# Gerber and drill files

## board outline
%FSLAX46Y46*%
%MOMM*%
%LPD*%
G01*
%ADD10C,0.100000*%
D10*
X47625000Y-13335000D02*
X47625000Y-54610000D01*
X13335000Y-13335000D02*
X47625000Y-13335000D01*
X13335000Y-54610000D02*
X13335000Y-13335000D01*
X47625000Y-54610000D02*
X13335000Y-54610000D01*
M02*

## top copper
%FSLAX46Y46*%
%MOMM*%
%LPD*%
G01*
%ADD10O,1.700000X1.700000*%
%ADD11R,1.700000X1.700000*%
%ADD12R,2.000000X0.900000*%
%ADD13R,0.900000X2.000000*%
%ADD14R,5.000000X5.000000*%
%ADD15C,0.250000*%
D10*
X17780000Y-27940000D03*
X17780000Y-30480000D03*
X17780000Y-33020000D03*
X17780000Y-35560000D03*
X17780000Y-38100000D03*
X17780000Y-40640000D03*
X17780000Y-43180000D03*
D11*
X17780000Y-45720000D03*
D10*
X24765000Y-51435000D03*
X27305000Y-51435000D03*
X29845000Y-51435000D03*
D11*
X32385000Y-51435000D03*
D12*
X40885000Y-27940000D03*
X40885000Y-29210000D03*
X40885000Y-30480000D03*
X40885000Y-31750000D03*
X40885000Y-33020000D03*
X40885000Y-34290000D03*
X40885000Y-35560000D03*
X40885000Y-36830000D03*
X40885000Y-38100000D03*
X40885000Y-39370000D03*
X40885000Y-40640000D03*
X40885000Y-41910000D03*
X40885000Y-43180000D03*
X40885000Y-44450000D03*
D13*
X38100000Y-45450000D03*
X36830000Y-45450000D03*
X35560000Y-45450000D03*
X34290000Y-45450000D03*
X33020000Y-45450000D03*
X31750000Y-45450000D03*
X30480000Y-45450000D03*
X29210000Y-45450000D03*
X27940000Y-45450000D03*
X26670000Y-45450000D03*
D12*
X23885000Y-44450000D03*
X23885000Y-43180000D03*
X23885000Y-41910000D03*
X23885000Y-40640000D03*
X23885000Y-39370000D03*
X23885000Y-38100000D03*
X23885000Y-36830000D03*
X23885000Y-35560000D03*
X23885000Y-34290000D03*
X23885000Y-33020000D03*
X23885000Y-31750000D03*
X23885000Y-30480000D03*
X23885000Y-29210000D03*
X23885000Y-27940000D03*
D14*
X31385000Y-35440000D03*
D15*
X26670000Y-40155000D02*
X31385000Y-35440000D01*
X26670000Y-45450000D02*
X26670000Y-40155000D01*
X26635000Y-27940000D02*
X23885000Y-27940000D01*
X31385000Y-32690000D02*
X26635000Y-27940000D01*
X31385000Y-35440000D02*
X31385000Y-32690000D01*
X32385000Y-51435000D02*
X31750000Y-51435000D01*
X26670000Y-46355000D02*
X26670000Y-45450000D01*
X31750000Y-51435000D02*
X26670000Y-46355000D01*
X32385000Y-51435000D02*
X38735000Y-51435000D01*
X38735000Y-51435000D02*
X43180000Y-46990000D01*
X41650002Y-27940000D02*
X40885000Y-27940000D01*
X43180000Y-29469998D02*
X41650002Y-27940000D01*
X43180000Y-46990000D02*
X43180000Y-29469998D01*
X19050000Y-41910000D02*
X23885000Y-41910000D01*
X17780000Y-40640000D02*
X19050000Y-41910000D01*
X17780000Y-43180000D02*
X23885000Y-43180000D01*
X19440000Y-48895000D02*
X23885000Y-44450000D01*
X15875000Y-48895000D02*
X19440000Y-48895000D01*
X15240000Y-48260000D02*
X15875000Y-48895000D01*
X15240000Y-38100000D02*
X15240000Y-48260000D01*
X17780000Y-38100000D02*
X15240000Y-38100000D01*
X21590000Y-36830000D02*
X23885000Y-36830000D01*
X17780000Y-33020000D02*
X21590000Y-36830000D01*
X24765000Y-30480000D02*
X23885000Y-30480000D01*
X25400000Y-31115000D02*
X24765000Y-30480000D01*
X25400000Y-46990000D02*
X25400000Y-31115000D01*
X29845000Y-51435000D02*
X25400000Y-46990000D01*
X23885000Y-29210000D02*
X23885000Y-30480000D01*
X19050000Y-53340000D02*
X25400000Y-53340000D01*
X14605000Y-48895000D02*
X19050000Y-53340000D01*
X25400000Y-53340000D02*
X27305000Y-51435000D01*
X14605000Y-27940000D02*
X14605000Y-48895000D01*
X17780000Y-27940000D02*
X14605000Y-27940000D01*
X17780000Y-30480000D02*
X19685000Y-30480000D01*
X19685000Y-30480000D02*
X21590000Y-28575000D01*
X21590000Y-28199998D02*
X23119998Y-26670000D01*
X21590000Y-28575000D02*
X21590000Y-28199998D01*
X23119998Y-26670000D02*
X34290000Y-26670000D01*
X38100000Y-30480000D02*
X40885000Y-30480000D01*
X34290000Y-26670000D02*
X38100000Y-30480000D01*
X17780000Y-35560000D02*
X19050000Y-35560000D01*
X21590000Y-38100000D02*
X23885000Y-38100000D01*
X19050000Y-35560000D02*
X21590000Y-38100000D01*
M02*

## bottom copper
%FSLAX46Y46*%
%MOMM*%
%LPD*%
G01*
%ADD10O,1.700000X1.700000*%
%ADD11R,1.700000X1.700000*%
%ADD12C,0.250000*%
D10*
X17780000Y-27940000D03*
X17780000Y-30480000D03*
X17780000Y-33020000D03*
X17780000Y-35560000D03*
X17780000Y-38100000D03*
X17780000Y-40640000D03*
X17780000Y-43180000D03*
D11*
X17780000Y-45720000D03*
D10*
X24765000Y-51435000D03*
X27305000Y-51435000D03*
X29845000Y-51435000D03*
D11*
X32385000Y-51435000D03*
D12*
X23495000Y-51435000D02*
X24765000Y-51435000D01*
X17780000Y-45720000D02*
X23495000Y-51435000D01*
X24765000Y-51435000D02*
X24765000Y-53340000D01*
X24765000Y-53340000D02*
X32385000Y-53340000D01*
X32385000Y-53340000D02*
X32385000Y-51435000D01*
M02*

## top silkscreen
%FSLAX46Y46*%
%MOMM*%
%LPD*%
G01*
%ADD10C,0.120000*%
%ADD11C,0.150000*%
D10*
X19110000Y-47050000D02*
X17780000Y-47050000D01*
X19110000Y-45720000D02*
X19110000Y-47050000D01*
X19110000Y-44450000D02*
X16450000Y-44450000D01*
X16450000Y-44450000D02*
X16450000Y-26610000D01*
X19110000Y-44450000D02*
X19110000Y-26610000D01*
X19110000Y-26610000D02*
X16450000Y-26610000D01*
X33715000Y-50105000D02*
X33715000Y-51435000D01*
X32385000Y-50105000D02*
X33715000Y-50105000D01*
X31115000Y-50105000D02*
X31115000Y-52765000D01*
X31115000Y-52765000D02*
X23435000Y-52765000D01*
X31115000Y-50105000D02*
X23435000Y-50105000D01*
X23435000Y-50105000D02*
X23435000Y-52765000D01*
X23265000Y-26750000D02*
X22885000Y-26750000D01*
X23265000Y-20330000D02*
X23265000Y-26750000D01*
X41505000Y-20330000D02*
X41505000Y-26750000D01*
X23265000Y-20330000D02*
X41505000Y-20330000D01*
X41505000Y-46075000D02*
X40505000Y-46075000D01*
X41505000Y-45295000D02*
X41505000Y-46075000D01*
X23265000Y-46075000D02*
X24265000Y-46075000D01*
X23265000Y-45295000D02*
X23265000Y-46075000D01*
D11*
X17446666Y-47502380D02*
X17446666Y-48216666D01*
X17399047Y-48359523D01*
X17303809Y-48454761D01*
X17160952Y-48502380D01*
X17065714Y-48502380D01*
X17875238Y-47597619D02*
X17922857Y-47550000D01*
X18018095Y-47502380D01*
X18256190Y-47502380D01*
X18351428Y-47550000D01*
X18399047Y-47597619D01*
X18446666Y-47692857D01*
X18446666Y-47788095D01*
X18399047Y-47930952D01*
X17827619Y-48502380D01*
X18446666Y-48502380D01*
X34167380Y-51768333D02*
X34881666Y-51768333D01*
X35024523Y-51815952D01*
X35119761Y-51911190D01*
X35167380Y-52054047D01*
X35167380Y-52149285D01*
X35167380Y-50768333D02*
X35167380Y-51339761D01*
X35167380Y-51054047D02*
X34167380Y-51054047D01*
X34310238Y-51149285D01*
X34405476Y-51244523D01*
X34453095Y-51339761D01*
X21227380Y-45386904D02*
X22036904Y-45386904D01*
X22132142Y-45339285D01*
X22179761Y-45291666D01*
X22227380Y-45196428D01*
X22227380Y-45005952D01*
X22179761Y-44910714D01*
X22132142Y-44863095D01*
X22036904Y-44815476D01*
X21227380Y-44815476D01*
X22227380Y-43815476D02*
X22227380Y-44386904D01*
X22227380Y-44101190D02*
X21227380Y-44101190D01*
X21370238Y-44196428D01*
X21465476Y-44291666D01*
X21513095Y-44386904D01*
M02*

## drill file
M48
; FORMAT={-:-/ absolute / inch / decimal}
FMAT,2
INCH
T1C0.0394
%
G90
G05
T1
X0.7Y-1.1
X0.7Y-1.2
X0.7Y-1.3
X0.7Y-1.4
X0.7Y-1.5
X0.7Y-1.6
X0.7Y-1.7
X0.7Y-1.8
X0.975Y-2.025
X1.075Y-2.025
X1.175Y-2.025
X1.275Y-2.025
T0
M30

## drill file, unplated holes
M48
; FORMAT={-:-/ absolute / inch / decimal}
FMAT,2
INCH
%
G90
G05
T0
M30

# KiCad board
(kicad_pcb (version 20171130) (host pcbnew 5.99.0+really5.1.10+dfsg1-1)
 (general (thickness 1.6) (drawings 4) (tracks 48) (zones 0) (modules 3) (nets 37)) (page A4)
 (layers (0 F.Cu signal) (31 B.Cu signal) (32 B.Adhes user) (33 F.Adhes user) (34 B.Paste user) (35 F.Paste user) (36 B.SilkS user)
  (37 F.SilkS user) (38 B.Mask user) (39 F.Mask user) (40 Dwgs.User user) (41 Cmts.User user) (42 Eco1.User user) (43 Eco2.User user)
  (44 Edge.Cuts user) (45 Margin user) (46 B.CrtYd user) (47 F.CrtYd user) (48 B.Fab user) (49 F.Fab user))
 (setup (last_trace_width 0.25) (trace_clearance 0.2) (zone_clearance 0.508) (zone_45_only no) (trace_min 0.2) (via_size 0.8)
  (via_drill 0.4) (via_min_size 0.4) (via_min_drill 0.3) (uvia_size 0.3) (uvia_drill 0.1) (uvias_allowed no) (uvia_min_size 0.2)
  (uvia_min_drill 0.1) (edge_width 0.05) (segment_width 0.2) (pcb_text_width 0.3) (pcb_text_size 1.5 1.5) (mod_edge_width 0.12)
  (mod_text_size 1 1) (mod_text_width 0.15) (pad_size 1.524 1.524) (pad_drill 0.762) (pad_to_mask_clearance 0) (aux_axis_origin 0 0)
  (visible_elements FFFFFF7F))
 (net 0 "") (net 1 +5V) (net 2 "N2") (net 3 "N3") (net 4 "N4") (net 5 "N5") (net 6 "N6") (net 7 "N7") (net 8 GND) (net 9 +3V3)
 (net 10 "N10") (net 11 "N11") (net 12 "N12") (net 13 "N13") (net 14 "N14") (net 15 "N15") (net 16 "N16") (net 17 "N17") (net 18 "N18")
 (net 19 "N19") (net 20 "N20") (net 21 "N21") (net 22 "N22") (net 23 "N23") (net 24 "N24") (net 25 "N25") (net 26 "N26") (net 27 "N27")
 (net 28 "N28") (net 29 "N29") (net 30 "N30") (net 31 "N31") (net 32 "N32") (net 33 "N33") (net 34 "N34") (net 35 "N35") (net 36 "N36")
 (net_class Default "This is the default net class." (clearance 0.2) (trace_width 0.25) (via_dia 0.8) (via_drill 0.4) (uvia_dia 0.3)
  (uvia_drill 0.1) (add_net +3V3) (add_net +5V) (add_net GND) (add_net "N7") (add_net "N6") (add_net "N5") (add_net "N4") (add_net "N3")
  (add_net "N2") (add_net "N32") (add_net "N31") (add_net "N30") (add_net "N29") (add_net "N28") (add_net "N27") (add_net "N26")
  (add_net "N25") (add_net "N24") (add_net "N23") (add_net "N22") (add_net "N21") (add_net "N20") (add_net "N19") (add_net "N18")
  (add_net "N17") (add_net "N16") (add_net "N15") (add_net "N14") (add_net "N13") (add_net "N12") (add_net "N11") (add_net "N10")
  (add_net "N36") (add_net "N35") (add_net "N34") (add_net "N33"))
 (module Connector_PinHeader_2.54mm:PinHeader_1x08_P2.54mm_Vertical (layer F.Cu) (at 17.78 45.72 180)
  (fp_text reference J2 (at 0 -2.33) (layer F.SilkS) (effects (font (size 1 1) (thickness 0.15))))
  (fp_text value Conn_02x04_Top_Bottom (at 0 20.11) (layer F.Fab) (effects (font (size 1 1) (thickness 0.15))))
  (fp_line (start -1.33 -1.33) (end 0 -1.33) (layer F.SilkS) (width 0.12))
  (fp_line (start -1.33 0) (end -1.33 -1.33) (layer F.SilkS) (width 0.12))
  (fp_line (start -1.33 1.27) (end 1.33 1.27) (layer F.SilkS) (width 0.12))
  (fp_line (start 1.33 1.27) (end 1.33 19.11) (layer F.SilkS) (width 0.12))
  (fp_line (start -1.33 1.27) (end -1.33 19.11) (layer F.SilkS) (width 0.12))
  (fp_line (start -1.33 19.11) (end 1.33 19.11) (layer F.SilkS) (width 0.12))
  (pad 8 thru_hole oval (at 0 17.78 180) (size 1.7 1.7) (drill 1) (layers *.Cu *.Mask) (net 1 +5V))
  (pad 7 thru_hole oval (at 0 15.24 180) (size 1.7 1.7) (drill 1) (layers *.Cu *.Mask) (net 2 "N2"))
  (pad 6 thru_hole oval (at 0 12.7 180) (size 1.7 1.7) (drill 1) (layers *.Cu *.Mask) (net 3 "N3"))
  (pad 5 thru_hole oval (at 0 10.16 180) (size 1.7 1.7) (drill 1) (layers *.Cu *.Mask) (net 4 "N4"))
  (pad 4 thru_hole oval (at 0 7.62 180) (size 1.7 1.7) (drill 1) (layers *.Cu *.Mask) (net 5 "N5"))
  (pad 3 thru_hole oval (at 0 5.08 180) (size 1.7 1.7) (drill 1) (layers *.Cu *.Mask) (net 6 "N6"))
  (pad 2 thru_hole oval (at 0 2.54 180) (size 1.7 1.7) (drill 1) (layers *.Cu *.Mask) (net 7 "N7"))
  (pad 1 thru_hole rect (at 0 0 180) (size 1.7 1.7) (drill 1) (layers *.Cu *.Mask) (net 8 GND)))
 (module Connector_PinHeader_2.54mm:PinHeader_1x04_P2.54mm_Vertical (layer F.Cu) (at 32.385 51.435 270)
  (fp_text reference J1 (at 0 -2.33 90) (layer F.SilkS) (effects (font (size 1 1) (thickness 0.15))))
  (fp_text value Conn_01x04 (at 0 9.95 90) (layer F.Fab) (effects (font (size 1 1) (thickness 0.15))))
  (fp_line (start -1.33 -1.33) (end 0 -1.33) (layer F.SilkS) (width 0.12))
  (fp_line (start -1.33 0) (end -1.33 -1.33) (layer F.SilkS) (width 0.12))
  (fp_line (start -1.33 1.27) (end 1.33 1.27) (layer F.SilkS) (width 0.12))
  (fp_line (start 1.33 1.27) (end 1.33 8.95) (layer F.SilkS) (width 0.12))
  (fp_line (start -1.33 1.27) (end -1.33 8.95) (layer F.SilkS) (width 0.12))
  (fp_line (start -1.33 8.95) (end 1.33 8.95) (layer F.SilkS) (width 0.12))
  (pad 4 thru_hole oval (at 0 7.62 270) (size 1.7 1.7) (drill 1) (layers *.Cu *.Mask) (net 8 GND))
  (pad 3 thru_hole oval (at 0 5.08 270) (size 1.7 1.7) (drill 1) (layers *.Cu *.Mask) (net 1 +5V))
  (pad 2 thru_hole oval (at 0 2.54 270) (size 1.7 1.7) (drill 1) (layers *.Cu *.Mask) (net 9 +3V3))
  (pad 1 thru_hole rect (at 0 0 270) (size 1.7 1.7) (drill 1) (layers *.Cu *.Mask) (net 8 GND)))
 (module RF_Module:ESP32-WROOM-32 (layer F.Cu) (at 32.385 36.195)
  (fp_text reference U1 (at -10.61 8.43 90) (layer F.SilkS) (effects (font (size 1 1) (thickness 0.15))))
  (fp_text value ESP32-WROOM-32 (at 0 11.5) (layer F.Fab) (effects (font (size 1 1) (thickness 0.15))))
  (fp_line (start -9.12 -9.445) (end -9.5 -9.445) (layer F.SilkS) (width 0.12))
  (fp_line (start -9.12 -15.865) (end -9.12 -9.445) (layer F.SilkS) (width 0.12))
  (fp_line (start 9.12 -15.865) (end 9.12 -9.445) (layer F.SilkS) (width 0.12))
  (fp_line (start -9.12 -15.865) (end 9.12 -15.865) (layer F.SilkS) (width 0.12))
  (fp_line (start 9.12 9.88) (end 8.12 9.88) (layer F.SilkS) (width 0.12))
  (fp_line (start 9.12 9.1) (end 9.12 9.88) (layer F.SilkS) (width 0.12))
  (fp_line (start -9.12 9.88) (end -8.12 9.88) (layer F.SilkS) (width 0.12))
  (fp_line (start -9.12 9.1) (end -9.12 9.88) (layer F.SilkS) (width 0.12))
  (pad 38 smd rect (at 8.5 -8.255) (size 2 0.9) (layers F.Cu F.Paste F.Mask) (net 8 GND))
  (pad 37 smd rect (at 8.5 -6.985) (size 2 0.9) (layers F.Cu F.Paste F.Mask) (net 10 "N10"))
  (pad 36 smd rect (at 8.5 -5.715) (size 2 0.9) (layers F.Cu F.Paste F.Mask) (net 2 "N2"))
  (pad 35 smd rect (at 8.5 -4.445) (size 2 0.9) (layers F.Cu F.Paste F.Mask) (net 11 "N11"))
  (pad 34 smd rect (at 8.5 -3.175) (size 2 0.9) (layers F.Cu F.Paste F.Mask) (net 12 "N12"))
  (pad 33 smd rect (at 8.5 -1.905) (size 2 0.9) (layers F.Cu F.Paste F.Mask) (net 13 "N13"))
  (pad 32 smd rect (at 8.5 -0.635) (size 2 0.9) (layers F.Cu F.Paste F.Mask) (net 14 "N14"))
  (pad 31 smd rect (at 8.5 0.635) (size 2 0.9) (layers F.Cu F.Paste F.Mask) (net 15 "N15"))
  (pad 30 smd rect (at 8.5 1.905) (size 2 0.9) (layers F.Cu F.Paste F.Mask) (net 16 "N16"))
  (pad 29 smd rect (at 8.5 3.175) (size 2 0.9) (layers F.Cu F.Paste F.Mask) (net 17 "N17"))
  (pad 28 smd rect (at 8.5 4.445) (size 2 0.9) (layers F.Cu F.Paste F.Mask) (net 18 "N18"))
  (pad 27 smd rect (at 8.5 5.715) (size 2 0.9) (layers F.Cu F.Paste F.Mask) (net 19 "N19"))
  (pad 26 smd rect (at 8.5 6.985) (size 2 0.9) (layers F.Cu F.Paste F.Mask) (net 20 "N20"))
  (pad 25 smd rect (at 8.5 8.255) (size 2 0.9) (layers F.Cu F.Paste F.Mask) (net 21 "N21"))
  (pad 24 smd rect (at 5.715 9.255 90) (size 2 0.9) (layers F.Cu F.Paste F.Mask) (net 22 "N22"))
  (pad 23 smd rect (at 4.445 9.255 90) (size 2 0.9) (layers F.Cu F.Paste F.Mask) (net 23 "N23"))
  (pad 22 smd rect (at 3.175 9.255 90) (size 2 0.9) (layers F.Cu F.Paste F.Mask) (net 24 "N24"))
  (pad 21 smd rect (at 1.905 9.255 90) (size 2 0.9) (layers F.Cu F.Paste F.Mask) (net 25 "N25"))
  (pad 20 smd rect (at 0.635 9.255 90) (size 2 0.9) (layers F.Cu F.Paste F.Mask) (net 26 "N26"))
  (pad 19 smd rect (at -0.635 9.255 90) (size 2 0.9) (layers F.Cu F.Paste F.Mask) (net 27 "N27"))
  (pad 18 smd rect (at -1.905 9.255 90) (size 2 0.9) (layers F.Cu F.Paste F.Mask) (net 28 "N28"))
  (pad 17 smd rect (at -3.175 9.255 90) (size 2 0.9) (layers F.Cu F.Paste F.Mask) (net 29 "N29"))
  (pad 16 smd rect (at -4.445 9.255 90) (size 2 0.9) (layers F.Cu F.Paste F.Mask) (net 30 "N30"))
  (pad 15 smd rect (at -5.715 9.255 90) (size 2 0.9) (layers F.Cu F.Paste F.Mask) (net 8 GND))
  (pad 14 smd rect (at -8.5 8.255) (size 2 0.9) (layers F.Cu F.Paste F.Mask) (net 5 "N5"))
  (pad 13 smd rect (at -8.5 6.985) (size 2 0.9) (layers F.Cu F.Paste F.Mask) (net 7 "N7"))
  (pad 12 smd rect (at -8.5 5.715) (size 2 0.9) (layers F.Cu F.Paste F.Mask) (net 6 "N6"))
  (pad 11 smd rect (at -8.5 4.445) (size 2 0.9) (layers F.Cu F.Paste F.Mask) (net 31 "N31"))
  (pad 10 smd rect (at -8.5 3.175) (size 2 0.9) (layers F.Cu F.Paste F.Mask) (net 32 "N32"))
  (pad 9 smd rect (at -8.5 1.905) (size 2 0.9) (layers F.Cu F.Paste F.Mask) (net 4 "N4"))
  (pad 8 smd rect (at -8.5 0.635) (size 2 0.9) (layers F.Cu F.Paste F.Mask) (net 3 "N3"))
  (pad 7 smd rect (at -8.5 -0.635) (size 2 0.9) (layers F.Cu F.Paste F.Mask) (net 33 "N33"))
  (pad 6 smd rect (at -8.5 -1.905) (size 2 0.9) (layers F.Cu F.Paste F.Mask) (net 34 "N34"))
  (pad 5 smd rect (at -8.5 -3.175) (size 2 0.9) (layers F.Cu F.Paste F.Mask) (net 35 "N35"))
  (pad 4 smd rect (at -8.5 -4.445) (size 2 0.9) (layers F.Cu F.Paste F.Mask) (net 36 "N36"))
  (pad 3 smd rect (at -8.5 -5.715) (size 2 0.9) (layers F.Cu F.Paste F.Mask) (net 9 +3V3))
  (pad 2 smd rect (at -8.5 -6.985) (size 2 0.9) (layers F.Cu F.Paste F.Mask) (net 9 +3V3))
  (pad 1 smd rect (at -8.5 -8.255) (size 2 0.9) (layers F.Cu F.Paste F.Mask) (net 8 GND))
  (pad 39 smd rect (at -1 -0.755) (size 5 5) (layers F.Cu F.Paste F.Mask) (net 8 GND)))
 (gr_line (start 47.625 13.335) (end 47.625 54.61) (layer Edge.Cuts) (width 0.1))
 (gr_line (start 13.335 13.335) (end 47.625 13.335) (layer Edge.Cuts) (width 0.1))
 (gr_line (start 13.335 54.61) (end 13.335 13.335) (layer Edge.Cuts) (width 0.1))
 (gr_line (start 47.625 54.61) (end 13.335 54.61) (layer Edge.Cuts) (width 0.1))
 (segment (start 23.495 51.435) (end 24.765 51.435) (width 0.25) (layer B.Cu) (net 8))
 (segment (start 17.78 45.72) (end 23.495 51.435) (width 0.25) (layer B.Cu) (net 8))
 (segment (start 24.765 51.435) (end 24.765 53.34) (width 0.25) (layer B.Cu) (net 8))
 (segment (start 24.765 53.34) (end 32.385 53.34) (width 0.25) (layer B.Cu) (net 8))
 (segment (start 32.385 53.34) (end 32.385 51.435) (width 0.25) (layer B.Cu) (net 8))
 (segment (start 26.67 40.155) (end 31.385 35.44) (width 0.25) (layer F.Cu) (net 8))
 (segment (start 26.67 45.45) (end 26.67 40.155) (width 0.25) (layer F.Cu) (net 8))
 (segment (start 26.635 27.94) (end 23.885 27.94) (width 0.25) (layer F.Cu) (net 8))
 (segment (start 31.385 32.69) (end 26.635 27.94) (width 0.25) (layer F.Cu) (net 8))
 (segment (start 31.385 35.44) (end 31.385 32.69) (width 0.25) (layer F.Cu) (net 8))
 (segment (start 32.385 51.435) (end 31.75 51.435) (width 0.25) (layer F.Cu) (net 8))
 (segment (start 26.67 46.355) (end 26.67 45.45) (width 0.25) (layer F.Cu) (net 8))
 (segment (start 31.75 51.435) (end 26.67 46.355) (width 0.25) (layer F.Cu) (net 8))
 (segment (start 32.385 51.435) (end 38.735 51.435) (width 0.25) (layer F.Cu) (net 8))
 (segment (start 38.735 51.435) (end 43.18 46.99) (width 0.25) (layer F.Cu) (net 8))
 (segment (start 41.650002 27.94) (end 40.885 27.94) (width 0.25) (layer F.Cu) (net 8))
 (segment (start 43.18 29.469998) (end 41.650002 27.94) (width 0.25) (layer F.Cu) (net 8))
 (segment (start 43.18 46.99) (end 43.18 29.469998) (width 0.25) (layer F.Cu) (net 8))
 (segment (start 19.05 41.91) (end 23.885 41.91) (width 0.25) (layer F.Cu) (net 6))
 (segment (start 17.78 40.64) (end 19.05 41.91) (width 0.25) (layer F.Cu) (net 6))
 (segment (start 17.78 43.18) (end 23.885 43.18) (width 0.25) (layer F.Cu) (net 7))
 (segment (start 19.44 48.895) (end 23.885 44.45) (width 0.25) (layer F.Cu) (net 5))
 (segment (start 15.875 48.895) (end 19.44 48.895) (width 0.25) (layer F.Cu) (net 5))
 (segment (start 15.24 48.26) (end 15.875 48.895) (width 0.25) (layer F.Cu) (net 5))
 (segment (start 15.24 38.1) (end 15.24 48.26) (width 0.25) (layer F.Cu) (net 5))
 (segment (start 17.78 38.1) (end 15.24 38.1) (width 0.25) (layer F.Cu) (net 5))
 (segment (start 21.59 36.83) (end 23.885 36.83) (width 0.25) (layer F.Cu) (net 3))
 (segment (start 17.78 33.02) (end 21.59 36.83) (width 0.25) (layer F.Cu) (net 3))
 (segment (start 24.765 30.48) (end 23.885 30.48) (width 0.25) (layer F.Cu) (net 9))
 (segment (start 25.4 31.115) (end 24.765 30.48) (width 0.25) (layer F.Cu) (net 9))
 (segment (start 25.4 46.99) (end 25.4 31.115) (width 0.25) (layer F.Cu) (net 9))
 (segment (start 29.845 51.435) (end 25.4 46.99) (width 0.25) (layer F.Cu) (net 9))
 (segment (start 23.885 29.21) (end 23.885 30.48) (width 0.25) (layer F.Cu) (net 9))
 (segment (start 19.05 53.34) (end 25.4 53.34) (width 0.25) (layer F.Cu) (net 1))
 (segment (start 14.605 48.895) (end 19.05 53.34) (width 0.25) (layer F.Cu) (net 1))
 (segment (start 25.4 53.34) (end 27.305 51.435) (width 0.25) (layer F.Cu) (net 1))
 (segment (start 14.605 27.94) (end 14.605 48.895) (width 0.25) (layer F.Cu) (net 1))
 (segment (start 17.78 27.94) (end 14.605 27.94) (width 0.25) (layer F.Cu) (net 1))
 (segment (start 17.78 30.48) (end 19.685 30.48) (width 0.25) (layer F.Cu) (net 2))
 (segment (start 19.685 30.48) (end 21.59 28.575) (width 0.25) (layer F.Cu) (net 2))
 (segment (start 21.59 28.199998) (end 23.119998 26.67) (width 0.25) (layer F.Cu) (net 2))
 (segment (start 21.59 28.575) (end 21.59 28.199998) (width 0.25) (layer F.Cu) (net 2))
 (segment (start 23.119998 26.67) (end 34.29 26.67) (width 0.25) (layer F.Cu) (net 2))
 (segment (start 38.1 30.48) (end 40.885 30.48) (width 0.25) (layer F.Cu) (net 2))
 (segment (start 34.29 26.67) (end 38.1 30.48) (width 0.25) (layer F.Cu) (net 2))
 (segment (start 17.78 35.56) (end 19.05 35.56) (width 0.25) (layer F.Cu) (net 4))
 (segment (start 21.59 38.1) (end 23.885 38.1) (width 0.25) (layer F.Cu) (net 4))
 (segment (start 19.05 35.56) (end 21.59 38.1) (width 0.25) (layer F.Cu) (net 4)))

